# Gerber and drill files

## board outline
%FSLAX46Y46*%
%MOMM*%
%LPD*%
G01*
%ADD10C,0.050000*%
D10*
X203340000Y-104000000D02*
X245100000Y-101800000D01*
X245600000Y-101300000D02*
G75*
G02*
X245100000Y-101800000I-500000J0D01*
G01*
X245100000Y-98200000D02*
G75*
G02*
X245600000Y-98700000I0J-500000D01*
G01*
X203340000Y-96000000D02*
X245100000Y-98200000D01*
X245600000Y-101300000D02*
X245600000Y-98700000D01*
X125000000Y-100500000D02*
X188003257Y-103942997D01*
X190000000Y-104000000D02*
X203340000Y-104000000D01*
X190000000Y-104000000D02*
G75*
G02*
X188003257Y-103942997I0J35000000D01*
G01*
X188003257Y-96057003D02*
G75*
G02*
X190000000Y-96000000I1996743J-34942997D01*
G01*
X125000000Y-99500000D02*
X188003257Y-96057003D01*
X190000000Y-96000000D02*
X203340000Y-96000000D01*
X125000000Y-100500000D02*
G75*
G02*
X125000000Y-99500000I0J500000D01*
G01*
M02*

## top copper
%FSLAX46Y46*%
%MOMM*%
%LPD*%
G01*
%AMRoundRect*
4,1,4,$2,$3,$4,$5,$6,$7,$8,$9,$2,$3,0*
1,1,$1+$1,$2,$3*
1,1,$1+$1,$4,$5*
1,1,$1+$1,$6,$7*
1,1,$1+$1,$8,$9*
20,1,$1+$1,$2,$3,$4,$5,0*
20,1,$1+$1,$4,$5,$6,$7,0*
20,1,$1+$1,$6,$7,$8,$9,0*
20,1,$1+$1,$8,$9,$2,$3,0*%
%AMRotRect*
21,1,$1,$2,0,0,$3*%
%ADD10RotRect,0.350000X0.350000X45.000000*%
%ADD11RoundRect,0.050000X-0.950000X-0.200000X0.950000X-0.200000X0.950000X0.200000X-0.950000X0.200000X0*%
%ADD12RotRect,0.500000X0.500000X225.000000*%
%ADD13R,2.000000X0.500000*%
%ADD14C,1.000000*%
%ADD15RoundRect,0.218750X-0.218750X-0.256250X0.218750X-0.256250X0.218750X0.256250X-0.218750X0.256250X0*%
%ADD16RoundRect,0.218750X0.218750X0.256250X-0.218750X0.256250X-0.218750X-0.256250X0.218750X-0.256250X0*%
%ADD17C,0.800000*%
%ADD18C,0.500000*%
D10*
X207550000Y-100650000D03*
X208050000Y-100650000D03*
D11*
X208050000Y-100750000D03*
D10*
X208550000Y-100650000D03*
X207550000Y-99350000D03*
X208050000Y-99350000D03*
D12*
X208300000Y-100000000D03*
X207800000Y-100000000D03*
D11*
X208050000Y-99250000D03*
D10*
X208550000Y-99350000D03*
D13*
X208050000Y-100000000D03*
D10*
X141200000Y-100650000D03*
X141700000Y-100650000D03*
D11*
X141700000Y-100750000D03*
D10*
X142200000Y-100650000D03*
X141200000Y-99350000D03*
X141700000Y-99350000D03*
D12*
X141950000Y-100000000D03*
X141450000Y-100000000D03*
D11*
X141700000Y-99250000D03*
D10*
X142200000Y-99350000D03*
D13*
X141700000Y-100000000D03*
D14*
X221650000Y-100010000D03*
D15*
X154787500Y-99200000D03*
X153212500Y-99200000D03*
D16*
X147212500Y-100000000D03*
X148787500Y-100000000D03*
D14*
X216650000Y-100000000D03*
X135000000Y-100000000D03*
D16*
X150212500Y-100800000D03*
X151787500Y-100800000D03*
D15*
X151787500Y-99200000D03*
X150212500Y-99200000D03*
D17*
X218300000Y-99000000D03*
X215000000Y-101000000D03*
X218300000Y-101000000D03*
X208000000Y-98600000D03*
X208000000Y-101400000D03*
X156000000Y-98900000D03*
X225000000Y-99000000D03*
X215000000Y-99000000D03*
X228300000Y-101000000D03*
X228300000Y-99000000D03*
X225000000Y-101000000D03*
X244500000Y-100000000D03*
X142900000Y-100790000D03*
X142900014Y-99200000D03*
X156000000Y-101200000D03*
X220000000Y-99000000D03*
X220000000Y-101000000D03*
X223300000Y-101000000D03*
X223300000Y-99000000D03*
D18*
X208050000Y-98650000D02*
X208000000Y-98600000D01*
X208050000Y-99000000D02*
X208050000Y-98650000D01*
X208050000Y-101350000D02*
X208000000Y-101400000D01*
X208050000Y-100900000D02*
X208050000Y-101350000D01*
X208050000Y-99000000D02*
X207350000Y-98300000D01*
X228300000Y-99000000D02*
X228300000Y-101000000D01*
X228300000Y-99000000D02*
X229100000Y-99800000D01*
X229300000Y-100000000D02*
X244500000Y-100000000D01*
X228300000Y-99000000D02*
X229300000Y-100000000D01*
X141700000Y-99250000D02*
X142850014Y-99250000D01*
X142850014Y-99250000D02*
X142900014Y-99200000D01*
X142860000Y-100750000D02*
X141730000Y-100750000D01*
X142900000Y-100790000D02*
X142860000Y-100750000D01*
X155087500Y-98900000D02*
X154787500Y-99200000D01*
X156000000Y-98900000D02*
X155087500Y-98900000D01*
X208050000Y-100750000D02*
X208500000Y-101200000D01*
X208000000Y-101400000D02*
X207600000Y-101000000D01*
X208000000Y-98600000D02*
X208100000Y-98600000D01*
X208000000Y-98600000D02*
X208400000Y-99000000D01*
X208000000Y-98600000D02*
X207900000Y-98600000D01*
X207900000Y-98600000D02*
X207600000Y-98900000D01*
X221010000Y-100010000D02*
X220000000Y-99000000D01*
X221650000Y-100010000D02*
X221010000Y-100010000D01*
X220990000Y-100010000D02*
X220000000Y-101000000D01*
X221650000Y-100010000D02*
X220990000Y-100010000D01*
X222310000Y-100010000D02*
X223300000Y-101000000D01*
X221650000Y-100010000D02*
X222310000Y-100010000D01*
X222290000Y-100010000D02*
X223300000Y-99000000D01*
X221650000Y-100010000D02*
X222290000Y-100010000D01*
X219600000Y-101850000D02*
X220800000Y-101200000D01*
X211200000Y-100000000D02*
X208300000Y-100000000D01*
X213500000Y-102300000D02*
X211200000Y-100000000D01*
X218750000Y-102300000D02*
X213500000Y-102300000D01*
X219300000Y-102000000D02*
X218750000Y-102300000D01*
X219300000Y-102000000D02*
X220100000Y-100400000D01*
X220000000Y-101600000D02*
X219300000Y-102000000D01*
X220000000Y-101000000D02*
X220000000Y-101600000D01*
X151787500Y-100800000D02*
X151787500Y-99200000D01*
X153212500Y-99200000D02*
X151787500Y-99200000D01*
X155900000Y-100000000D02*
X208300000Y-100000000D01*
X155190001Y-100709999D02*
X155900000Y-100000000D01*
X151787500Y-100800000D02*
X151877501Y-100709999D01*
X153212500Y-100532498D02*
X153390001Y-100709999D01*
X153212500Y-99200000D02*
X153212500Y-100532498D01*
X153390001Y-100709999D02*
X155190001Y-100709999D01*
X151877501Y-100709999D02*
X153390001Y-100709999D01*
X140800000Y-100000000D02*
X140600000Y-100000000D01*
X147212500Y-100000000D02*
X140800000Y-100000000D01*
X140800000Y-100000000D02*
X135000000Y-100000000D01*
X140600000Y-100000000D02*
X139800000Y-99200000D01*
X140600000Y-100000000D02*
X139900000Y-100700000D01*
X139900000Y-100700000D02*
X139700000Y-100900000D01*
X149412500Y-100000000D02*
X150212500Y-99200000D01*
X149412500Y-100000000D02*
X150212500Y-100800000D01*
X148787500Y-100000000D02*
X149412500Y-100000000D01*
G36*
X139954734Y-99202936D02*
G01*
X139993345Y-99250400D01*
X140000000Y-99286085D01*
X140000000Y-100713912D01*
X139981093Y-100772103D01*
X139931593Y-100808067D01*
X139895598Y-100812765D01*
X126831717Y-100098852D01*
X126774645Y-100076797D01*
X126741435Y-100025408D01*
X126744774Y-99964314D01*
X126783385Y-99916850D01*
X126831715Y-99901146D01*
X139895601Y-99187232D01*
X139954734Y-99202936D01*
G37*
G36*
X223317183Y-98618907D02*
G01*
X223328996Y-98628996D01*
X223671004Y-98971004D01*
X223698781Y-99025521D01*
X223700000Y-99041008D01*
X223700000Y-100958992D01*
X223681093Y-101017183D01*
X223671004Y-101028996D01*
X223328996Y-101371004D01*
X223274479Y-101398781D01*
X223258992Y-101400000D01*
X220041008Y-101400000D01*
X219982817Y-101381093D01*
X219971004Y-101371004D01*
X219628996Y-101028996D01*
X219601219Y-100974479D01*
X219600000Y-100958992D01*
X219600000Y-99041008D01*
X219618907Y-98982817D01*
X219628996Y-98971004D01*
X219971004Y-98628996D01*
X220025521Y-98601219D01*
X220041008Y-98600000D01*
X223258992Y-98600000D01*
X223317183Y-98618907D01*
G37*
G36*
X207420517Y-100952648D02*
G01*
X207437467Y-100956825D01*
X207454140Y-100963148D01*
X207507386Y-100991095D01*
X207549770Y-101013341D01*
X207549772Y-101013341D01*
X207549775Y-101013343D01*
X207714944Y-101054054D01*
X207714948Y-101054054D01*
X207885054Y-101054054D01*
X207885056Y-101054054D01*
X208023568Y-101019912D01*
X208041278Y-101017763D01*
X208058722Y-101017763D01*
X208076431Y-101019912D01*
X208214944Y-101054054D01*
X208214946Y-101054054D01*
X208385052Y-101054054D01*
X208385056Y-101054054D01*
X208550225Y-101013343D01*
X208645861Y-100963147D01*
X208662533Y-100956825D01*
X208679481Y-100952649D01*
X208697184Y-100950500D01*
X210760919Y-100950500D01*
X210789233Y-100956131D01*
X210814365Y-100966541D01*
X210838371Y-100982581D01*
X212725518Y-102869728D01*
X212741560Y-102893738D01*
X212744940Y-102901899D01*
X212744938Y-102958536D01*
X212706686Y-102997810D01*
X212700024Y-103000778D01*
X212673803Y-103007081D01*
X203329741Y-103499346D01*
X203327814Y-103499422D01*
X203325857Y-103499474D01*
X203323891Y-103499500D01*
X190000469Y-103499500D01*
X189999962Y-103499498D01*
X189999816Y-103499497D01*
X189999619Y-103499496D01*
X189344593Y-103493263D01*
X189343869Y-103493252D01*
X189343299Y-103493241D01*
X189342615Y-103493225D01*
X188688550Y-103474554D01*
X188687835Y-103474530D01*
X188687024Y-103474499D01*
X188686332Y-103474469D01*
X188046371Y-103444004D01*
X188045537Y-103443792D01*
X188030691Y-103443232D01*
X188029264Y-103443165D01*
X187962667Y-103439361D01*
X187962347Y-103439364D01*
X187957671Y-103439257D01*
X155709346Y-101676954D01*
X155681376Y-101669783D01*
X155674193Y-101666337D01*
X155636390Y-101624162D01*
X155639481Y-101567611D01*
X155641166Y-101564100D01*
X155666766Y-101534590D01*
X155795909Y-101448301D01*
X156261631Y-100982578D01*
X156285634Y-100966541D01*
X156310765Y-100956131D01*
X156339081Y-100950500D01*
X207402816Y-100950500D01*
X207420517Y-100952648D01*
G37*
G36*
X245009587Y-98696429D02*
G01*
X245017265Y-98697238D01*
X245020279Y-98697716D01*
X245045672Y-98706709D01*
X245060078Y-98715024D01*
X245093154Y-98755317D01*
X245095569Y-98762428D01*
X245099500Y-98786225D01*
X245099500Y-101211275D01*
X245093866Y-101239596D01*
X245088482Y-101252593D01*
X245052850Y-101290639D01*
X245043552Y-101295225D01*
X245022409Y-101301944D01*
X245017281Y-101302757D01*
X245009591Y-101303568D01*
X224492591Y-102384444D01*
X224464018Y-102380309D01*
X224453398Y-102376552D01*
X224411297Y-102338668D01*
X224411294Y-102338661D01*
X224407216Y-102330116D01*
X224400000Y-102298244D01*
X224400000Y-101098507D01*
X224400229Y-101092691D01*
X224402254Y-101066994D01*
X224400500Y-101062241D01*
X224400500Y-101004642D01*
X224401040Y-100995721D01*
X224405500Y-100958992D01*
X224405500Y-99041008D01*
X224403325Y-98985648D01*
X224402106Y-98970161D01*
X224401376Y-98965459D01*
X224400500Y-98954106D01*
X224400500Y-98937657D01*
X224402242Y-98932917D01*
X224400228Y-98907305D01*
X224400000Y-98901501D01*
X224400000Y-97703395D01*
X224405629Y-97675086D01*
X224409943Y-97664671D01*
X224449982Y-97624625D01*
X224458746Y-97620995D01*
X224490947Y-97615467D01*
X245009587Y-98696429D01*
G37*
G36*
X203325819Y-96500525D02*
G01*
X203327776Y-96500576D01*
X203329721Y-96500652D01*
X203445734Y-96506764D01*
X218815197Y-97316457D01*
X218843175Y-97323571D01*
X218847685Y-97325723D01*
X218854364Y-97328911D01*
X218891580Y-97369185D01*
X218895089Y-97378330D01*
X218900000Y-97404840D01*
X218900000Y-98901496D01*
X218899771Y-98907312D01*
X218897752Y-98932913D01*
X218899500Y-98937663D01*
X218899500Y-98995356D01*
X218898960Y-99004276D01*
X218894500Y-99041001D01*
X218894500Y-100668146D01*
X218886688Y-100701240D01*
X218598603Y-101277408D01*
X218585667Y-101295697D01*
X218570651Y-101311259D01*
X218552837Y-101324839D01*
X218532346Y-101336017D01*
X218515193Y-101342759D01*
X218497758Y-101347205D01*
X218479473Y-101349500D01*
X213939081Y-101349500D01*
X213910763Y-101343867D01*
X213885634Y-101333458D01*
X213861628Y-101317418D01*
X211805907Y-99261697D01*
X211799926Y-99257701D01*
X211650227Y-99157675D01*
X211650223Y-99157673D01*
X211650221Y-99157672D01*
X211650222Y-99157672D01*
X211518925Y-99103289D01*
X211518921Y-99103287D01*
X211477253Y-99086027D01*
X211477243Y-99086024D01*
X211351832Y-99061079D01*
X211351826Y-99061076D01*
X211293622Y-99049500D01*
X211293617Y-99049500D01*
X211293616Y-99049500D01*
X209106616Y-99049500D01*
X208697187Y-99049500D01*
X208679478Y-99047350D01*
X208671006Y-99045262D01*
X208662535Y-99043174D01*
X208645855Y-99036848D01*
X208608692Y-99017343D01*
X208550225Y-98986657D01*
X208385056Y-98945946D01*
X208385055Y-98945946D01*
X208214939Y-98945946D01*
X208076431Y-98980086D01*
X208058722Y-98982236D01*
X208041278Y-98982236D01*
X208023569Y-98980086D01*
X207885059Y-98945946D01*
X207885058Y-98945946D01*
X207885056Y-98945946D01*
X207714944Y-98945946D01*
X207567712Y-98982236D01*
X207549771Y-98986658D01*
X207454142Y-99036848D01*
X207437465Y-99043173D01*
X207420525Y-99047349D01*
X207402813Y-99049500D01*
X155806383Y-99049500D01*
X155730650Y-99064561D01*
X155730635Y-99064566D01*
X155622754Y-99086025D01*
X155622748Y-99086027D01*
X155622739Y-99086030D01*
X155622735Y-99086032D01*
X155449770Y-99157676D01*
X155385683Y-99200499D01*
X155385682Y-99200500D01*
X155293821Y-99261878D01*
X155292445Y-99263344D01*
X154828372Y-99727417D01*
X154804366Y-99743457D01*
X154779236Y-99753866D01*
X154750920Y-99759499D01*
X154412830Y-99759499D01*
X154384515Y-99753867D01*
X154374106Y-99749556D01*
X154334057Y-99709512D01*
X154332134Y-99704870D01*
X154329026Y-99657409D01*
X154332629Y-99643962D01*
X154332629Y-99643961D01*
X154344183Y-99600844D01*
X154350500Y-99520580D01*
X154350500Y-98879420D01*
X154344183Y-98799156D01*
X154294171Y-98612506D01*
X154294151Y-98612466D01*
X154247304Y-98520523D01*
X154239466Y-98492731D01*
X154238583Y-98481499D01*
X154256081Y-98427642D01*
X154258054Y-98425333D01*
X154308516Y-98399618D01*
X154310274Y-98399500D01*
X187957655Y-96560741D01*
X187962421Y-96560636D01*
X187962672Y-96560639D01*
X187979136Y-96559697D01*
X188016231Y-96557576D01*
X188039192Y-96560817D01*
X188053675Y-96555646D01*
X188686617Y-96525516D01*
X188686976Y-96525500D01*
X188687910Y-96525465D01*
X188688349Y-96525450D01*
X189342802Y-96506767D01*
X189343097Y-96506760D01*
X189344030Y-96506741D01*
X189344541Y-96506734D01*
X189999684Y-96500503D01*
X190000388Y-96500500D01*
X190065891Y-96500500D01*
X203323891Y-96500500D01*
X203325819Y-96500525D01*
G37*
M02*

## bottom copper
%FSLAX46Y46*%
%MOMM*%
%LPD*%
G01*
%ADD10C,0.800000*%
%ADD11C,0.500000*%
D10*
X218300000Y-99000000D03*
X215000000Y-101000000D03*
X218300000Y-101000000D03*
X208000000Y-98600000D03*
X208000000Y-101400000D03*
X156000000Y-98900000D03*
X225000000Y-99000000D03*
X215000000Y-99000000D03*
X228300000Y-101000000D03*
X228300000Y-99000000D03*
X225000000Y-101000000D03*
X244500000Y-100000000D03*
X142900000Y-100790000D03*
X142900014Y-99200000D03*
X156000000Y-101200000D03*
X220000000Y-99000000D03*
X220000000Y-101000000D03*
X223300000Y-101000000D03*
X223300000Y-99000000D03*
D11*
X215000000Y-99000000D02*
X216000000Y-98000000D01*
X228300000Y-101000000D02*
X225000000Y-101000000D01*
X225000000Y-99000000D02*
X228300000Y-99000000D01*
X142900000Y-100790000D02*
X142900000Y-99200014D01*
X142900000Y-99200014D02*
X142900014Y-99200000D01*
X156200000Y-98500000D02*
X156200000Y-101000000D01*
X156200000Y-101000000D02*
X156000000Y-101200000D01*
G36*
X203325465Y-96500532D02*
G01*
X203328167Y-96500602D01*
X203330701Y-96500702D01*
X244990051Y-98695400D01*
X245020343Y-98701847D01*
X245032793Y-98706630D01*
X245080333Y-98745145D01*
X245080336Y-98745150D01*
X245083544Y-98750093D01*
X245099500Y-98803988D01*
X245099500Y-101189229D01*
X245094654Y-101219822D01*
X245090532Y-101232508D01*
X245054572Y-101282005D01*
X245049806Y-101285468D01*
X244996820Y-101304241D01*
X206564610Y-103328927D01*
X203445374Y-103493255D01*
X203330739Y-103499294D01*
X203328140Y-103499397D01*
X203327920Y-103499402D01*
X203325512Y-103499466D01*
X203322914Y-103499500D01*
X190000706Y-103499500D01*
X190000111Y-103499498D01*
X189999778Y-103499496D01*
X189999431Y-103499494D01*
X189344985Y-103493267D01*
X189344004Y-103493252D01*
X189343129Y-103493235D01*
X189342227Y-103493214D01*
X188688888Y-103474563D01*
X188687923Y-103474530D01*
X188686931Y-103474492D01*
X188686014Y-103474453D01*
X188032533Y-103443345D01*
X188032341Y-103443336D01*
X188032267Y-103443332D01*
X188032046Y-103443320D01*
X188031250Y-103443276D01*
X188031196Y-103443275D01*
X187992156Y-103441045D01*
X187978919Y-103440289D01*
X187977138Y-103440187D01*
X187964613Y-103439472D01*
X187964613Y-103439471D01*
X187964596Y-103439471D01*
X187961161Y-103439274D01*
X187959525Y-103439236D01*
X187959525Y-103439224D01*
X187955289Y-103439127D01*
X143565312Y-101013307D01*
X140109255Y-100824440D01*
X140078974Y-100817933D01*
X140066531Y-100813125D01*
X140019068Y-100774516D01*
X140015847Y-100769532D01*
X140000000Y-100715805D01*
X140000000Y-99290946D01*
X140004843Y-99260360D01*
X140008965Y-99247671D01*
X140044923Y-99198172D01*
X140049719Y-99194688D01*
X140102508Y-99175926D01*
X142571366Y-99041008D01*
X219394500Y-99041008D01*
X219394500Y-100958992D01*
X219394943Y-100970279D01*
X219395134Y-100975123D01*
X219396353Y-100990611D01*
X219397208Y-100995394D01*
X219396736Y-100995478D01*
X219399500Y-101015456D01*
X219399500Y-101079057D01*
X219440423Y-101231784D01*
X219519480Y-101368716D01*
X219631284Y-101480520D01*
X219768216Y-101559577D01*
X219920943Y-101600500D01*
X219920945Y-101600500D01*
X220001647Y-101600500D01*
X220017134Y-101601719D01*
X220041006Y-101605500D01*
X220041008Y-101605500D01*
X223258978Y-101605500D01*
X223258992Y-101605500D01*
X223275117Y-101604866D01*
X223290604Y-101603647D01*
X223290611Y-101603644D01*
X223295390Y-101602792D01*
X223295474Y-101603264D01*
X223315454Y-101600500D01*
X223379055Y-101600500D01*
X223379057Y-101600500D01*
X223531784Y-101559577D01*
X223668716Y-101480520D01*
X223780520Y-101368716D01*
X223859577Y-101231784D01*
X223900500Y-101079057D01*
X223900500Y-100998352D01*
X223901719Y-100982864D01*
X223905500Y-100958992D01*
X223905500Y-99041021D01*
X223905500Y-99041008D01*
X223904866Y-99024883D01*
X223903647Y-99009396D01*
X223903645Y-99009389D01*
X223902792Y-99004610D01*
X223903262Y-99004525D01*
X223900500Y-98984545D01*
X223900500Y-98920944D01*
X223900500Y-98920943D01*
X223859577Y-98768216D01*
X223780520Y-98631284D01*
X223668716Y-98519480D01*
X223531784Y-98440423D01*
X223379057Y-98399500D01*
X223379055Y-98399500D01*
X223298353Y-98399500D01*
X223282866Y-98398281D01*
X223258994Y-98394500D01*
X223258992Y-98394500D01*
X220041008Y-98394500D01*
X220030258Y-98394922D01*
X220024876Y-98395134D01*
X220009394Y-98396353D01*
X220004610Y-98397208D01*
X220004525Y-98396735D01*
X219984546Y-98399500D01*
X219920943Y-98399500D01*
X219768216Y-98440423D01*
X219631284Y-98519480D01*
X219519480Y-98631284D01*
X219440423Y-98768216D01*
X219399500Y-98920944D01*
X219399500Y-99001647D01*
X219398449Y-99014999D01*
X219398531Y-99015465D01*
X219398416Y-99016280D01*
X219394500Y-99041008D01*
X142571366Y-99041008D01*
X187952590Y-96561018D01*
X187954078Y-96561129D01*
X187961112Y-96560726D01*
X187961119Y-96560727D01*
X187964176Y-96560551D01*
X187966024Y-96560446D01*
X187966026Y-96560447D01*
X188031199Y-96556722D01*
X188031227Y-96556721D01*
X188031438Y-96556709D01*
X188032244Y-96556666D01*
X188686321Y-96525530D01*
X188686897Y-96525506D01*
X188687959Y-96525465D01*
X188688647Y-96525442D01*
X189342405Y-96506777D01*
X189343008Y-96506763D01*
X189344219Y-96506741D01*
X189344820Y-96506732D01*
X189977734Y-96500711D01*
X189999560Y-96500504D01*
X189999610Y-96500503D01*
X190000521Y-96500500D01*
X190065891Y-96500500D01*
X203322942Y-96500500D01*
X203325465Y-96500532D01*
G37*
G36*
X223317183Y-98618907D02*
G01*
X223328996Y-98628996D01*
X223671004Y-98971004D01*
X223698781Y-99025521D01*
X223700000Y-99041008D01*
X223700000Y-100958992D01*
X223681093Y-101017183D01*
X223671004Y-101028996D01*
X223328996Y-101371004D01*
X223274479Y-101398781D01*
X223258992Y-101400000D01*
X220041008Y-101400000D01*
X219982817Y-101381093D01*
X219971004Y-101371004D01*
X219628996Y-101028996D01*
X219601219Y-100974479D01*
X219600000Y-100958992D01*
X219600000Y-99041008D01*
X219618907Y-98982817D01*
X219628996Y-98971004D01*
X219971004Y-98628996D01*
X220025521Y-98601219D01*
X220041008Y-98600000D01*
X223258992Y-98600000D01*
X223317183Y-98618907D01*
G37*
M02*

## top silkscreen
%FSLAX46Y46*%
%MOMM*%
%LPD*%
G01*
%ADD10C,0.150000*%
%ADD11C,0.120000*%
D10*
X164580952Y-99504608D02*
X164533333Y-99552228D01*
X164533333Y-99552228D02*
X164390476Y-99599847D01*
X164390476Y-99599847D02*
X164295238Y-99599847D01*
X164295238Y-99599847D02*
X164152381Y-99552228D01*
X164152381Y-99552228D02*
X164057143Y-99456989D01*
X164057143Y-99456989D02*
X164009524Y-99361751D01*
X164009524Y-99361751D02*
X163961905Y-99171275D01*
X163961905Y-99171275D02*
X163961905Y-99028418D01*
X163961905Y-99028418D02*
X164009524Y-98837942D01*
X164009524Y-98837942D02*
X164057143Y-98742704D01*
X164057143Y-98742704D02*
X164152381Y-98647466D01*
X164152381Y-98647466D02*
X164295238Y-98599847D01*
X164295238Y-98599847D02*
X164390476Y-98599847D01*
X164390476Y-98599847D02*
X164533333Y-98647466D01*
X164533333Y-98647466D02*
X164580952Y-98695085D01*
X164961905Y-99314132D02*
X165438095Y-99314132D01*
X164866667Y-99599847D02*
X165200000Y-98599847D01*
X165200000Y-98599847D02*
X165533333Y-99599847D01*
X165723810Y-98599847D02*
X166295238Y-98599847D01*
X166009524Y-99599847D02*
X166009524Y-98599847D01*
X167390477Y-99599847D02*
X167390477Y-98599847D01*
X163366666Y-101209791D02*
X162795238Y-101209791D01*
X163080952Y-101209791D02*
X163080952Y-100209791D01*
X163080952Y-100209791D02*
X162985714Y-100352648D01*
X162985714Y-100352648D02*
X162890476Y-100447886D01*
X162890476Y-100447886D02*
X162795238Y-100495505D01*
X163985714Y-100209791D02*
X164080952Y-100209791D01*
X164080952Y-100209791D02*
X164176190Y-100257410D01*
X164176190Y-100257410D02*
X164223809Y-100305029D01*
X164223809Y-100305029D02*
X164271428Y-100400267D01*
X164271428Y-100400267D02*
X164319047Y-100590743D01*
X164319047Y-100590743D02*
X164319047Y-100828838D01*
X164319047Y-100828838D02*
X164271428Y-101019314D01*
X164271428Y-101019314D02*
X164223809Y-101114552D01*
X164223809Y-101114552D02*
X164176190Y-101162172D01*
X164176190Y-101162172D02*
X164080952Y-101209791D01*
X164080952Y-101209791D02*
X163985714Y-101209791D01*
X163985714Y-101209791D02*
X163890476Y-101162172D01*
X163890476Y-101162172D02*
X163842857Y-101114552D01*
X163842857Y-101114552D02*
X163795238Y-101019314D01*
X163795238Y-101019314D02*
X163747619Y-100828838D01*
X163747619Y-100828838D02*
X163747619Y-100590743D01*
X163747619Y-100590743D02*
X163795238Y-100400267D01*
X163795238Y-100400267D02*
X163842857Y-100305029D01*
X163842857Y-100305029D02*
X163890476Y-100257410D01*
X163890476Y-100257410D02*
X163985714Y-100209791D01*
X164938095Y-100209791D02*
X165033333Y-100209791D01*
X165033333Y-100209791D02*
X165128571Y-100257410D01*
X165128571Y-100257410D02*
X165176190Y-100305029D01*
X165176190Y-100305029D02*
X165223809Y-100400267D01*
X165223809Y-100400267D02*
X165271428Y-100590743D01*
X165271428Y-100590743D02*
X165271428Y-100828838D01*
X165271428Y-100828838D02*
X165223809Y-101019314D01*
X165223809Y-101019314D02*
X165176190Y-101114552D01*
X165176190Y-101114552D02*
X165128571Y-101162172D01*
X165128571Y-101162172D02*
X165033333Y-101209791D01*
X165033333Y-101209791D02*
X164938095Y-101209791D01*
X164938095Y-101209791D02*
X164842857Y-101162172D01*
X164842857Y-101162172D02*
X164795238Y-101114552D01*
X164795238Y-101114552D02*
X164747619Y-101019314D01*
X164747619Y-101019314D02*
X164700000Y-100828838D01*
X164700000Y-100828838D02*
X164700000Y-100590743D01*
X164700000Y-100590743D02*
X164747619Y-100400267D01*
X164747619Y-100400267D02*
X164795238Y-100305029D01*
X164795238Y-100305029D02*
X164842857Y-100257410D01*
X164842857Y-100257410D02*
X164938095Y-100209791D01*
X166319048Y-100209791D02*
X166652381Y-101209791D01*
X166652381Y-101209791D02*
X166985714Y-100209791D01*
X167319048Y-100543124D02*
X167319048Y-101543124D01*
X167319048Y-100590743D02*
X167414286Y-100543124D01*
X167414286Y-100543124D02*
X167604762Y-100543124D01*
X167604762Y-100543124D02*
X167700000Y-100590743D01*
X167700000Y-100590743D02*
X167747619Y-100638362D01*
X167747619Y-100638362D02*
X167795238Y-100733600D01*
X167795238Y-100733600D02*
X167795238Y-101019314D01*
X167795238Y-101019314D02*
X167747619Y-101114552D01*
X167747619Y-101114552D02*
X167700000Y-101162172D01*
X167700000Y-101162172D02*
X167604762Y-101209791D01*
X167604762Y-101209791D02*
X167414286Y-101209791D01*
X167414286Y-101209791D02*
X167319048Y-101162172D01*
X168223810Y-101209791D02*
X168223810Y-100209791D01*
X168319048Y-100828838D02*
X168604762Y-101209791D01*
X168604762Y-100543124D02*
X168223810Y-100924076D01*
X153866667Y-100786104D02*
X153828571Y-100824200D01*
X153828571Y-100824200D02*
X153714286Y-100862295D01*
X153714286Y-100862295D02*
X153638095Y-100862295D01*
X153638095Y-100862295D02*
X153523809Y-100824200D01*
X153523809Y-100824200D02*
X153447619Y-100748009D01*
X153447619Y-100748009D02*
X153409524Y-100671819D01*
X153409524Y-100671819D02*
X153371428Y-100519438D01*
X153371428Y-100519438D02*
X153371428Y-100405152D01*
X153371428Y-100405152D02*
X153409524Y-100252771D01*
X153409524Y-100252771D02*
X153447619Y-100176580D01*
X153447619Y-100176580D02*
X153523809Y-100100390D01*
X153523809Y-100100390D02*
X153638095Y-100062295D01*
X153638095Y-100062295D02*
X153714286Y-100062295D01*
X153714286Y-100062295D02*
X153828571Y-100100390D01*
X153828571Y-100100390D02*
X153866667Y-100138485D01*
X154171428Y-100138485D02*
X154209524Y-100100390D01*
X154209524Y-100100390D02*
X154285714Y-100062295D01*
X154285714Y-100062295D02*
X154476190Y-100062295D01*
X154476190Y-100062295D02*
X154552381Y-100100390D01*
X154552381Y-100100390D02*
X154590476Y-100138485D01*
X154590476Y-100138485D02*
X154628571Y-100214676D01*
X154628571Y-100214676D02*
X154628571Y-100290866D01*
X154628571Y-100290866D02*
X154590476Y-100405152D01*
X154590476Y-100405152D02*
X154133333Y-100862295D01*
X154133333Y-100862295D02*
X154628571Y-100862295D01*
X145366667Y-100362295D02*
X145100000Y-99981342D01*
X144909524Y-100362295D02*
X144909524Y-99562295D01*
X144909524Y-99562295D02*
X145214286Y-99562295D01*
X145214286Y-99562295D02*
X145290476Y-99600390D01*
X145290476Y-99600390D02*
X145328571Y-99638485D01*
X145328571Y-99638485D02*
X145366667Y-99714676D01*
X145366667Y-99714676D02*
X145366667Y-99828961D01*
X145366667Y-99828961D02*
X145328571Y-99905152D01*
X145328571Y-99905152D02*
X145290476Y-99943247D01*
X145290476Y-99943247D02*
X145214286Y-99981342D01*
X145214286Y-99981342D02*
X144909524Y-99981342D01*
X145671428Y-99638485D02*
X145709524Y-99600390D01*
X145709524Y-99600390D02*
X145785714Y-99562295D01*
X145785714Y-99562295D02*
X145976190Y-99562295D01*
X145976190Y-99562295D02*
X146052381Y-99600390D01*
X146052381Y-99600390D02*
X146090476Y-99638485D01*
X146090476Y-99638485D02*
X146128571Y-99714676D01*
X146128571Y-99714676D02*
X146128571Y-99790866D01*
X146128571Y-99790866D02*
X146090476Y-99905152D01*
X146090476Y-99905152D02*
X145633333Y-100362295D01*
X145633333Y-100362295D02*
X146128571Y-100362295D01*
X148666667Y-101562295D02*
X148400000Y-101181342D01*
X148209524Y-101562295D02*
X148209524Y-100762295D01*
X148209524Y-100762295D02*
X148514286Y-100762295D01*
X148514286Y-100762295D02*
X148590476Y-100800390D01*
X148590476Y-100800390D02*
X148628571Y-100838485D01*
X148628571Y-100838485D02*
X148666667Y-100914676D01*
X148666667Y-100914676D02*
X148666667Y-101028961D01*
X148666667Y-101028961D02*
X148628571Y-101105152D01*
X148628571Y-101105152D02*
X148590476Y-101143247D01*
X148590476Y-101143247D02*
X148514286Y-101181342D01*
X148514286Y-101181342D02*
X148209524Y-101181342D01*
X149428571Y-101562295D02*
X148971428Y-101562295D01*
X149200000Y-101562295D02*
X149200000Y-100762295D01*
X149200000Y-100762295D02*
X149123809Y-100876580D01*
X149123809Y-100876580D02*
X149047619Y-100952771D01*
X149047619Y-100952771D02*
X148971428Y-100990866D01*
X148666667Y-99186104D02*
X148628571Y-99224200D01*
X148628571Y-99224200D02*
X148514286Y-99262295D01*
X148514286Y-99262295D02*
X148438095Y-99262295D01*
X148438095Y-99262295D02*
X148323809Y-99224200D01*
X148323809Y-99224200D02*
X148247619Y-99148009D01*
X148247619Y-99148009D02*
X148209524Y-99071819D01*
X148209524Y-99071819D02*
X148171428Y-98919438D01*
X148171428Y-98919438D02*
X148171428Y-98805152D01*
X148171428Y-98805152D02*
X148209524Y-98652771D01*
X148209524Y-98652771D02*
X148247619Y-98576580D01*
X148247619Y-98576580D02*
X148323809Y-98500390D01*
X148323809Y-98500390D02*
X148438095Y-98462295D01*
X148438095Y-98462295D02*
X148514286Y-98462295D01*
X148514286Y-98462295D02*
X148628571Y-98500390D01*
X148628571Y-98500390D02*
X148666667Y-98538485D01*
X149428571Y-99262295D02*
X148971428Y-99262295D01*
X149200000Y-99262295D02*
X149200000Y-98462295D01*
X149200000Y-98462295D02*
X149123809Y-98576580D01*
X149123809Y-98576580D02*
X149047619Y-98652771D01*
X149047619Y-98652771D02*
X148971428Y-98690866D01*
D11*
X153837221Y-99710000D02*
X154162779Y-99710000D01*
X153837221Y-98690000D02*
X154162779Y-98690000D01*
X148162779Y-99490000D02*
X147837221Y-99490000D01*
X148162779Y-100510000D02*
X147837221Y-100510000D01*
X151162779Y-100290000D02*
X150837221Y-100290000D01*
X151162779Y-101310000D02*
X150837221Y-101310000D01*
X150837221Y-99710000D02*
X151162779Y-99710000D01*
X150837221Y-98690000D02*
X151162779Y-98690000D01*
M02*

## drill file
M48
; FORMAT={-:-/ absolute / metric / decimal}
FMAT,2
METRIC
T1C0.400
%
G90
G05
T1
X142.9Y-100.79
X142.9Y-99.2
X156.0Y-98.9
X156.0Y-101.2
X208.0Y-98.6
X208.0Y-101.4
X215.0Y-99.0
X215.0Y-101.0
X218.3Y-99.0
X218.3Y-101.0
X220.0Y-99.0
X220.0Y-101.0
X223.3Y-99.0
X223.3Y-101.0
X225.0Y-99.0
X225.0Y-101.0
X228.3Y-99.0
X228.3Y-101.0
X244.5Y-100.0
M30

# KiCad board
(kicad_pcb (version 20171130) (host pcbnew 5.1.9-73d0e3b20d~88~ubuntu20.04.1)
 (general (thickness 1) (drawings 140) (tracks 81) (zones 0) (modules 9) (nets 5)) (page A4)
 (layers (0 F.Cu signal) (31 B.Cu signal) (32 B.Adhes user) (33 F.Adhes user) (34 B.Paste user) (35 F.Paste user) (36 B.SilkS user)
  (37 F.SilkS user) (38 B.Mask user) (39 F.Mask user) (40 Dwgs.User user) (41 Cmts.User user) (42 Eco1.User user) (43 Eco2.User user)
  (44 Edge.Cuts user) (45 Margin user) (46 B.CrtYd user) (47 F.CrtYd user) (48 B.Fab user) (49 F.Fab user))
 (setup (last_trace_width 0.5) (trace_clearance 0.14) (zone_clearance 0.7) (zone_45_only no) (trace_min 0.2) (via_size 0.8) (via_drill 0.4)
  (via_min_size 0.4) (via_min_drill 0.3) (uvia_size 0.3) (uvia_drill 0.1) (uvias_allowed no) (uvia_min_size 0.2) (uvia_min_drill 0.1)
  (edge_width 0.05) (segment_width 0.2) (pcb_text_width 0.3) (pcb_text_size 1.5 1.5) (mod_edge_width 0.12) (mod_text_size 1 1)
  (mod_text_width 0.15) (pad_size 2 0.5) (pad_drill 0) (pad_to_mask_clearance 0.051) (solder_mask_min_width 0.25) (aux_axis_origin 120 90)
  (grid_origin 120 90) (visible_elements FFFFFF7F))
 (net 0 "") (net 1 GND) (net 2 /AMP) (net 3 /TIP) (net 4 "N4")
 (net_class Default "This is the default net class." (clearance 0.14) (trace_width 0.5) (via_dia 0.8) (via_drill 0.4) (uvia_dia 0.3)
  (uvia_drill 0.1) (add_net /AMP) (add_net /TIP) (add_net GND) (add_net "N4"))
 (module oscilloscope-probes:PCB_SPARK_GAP (layer F.Cu) (at 208.05 100)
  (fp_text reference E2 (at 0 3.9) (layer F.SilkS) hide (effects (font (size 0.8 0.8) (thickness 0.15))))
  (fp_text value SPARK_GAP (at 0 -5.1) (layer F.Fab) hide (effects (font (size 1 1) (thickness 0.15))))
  (pad 2 smd rect (at -0.5 0.65 45) (size 0.35 0.35) (layers F.Cu) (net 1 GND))
  (pad 2 smd rect (at 0 0.65 45) (size 0.35 0.35) (layers F.Cu) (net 1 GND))
  (pad 2 smd roundrect (at 0 0.75) (size 2 0.5) (layers F.Cu) (roundrect_rratio 0.1) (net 1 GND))
  (pad 2 smd rect (at 0.5 0.65 45) (size 0.35 0.35) (layers F.Cu) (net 1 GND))
  (pad 2 smd rect (at -0.5 -0.65 45) (size 0.35 0.35) (layers F.Cu) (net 1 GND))
  (pad 2 smd rect (at 0 -0.65 45) (size 0.35 0.35) (layers F.Cu) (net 1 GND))
  (pad 1 smd rect (at 0.25 0 225) (size 0.5 0.5) (layers F.Cu F.Mask) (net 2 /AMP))
  (pad 1 smd rect (at -0.25 0 225) (size 0.5 0.5) (layers F.Cu F.Mask) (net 2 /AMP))
  (pad 2 smd roundrect (at 0 -0.75) (size 2 0.5) (layers F.Cu) (roundrect_rratio 0.1) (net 1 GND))
  (pad 2 smd rect (at 0.5 -0.65 45) (size 0.35 0.35) (layers F.Cu) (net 1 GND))
  (pad 1 smd rect (at 0 0) (size 2 0.5) (layers F.Cu F.Mask) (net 2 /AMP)))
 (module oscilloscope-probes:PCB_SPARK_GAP (layer F.Cu) (at 141.7 100)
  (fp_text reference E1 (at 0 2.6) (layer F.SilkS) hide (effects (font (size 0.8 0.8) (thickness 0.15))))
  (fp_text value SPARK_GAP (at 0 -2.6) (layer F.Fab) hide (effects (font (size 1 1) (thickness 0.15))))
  (pad 2 smd rect (at -0.5 0.65 45) (size 0.35 0.35) (layers F.Cu) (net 1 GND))
  (pad 2 smd rect (at 0 0.65 45) (size 0.35 0.35) (layers F.Cu) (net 1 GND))
  (pad 2 smd roundrect (at 0 0.75) (size 2 0.5) (layers F.Cu) (roundrect_rratio 0.1) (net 1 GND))
  (pad 2 smd rect (at 0.5 0.65 45) (size 0.35 0.35) (layers F.Cu) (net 1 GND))
  (pad 2 smd rect (at -0.5 -0.65 45) (size 0.35 0.35) (layers F.Cu) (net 1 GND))
  (pad 2 smd rect (at 0 -0.65 45) (size 0.35 0.35) (layers F.Cu) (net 1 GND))
  (pad 1 smd rect (at 0.25 0 225) (size 0.5 0.5) (layers F.Cu F.Mask) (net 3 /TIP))
  (pad 1 smd rect (at -0.25 0 225) (size 0.5 0.5) (layers F.Cu F.Mask) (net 3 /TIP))
  (pad 2 smd roundrect (at 0 -0.75) (size 2 0.5) (layers F.Cu) (roundrect_rratio 0.1) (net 1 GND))
  (pad 2 smd rect (at 0.5 -0.65 45) (size 0.35 0.35) (layers F.Cu) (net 1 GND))
  (pad 1 smd rect (at 0 0) (size 2 0.5) (layers F.Cu F.Mask) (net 3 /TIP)))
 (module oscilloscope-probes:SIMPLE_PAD (layer F.Cu) (at 221.65 100.01)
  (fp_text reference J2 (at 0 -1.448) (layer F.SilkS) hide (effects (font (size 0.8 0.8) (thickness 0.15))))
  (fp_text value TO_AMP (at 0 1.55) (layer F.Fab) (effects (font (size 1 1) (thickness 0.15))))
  (pad 1 smd circle (at 0 0) (size 1 1) (layers F.Cu F.Mask) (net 2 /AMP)))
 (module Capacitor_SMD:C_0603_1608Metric (layer F.Cu) (at 154 99.2)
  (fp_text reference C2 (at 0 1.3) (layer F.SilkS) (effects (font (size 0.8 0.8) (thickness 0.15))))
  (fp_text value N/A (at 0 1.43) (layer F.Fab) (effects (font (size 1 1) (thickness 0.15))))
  (fp_line (start -0.162779 0.51) (end 0.162779 0.51) (layer F.SilkS) (width 0.12))
  (fp_line (start -0.162779 -0.51) (end 0.162779 -0.51) (layer F.SilkS) (width 0.12))
  (pad 2 smd roundrect (at 0.7875 0) (size 0.875 0.95) (layers F.Cu F.Paste F.Mask) (roundrect_rratio 0.25) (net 1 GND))
  (pad 1 smd roundrect (at -0.7875 0) (size 0.875 0.95) (layers F.Cu F.Paste F.Mask) (roundrect_rratio 0.25) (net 2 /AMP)))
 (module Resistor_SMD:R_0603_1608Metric (layer F.Cu) (at 148 100 180)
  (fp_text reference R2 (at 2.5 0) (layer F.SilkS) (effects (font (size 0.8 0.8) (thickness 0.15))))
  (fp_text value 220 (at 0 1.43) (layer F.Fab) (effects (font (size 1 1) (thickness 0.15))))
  (fp_line (start -0.162779 0.51) (end 0.162779 0.51) (layer F.SilkS) (width 0.12))
  (fp_line (start -0.162779 -0.51) (end 0.162779 -0.51) (layer F.SilkS) (width 0.12))
  (pad 2 smd roundrect (at 0.7875 0 180) (size 0.875 0.95) (layers F.Cu F.Paste F.Mask) (roundrect_rratio 0.25) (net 3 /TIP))
  (pad 1 smd roundrect (at -0.7875 0 180) (size 0.875 0.95) (layers F.Cu F.Paste F.Mask) (roundrect_rratio 0.25) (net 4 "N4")))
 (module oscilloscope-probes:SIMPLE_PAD (layer F.Cu) (at 216.65 100)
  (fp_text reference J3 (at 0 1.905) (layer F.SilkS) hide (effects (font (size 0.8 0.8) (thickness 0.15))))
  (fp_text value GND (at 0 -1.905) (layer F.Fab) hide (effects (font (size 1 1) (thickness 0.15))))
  (pad 1 smd circle (at 0 0) (size 1 1) (layers F.Cu F.Mask) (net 1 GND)))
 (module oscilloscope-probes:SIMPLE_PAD (layer F.Cu) (at 135 100)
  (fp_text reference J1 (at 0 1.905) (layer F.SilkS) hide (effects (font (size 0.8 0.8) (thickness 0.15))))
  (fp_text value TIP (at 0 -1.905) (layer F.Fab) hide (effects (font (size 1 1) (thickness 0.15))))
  (pad 1 smd circle (at 0 0) (size 1 1) (layers F.Cu F.Mask) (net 3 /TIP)))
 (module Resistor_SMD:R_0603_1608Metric (layer F.Cu) (at 151 100.8 180)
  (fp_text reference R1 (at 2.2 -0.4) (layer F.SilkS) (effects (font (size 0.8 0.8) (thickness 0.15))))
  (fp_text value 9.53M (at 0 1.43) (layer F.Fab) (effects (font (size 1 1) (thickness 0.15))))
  (fp_line (start -0.162779 0.51) (end 0.162779 0.51) (layer F.SilkS) (width 0.12))
  (fp_line (start -0.162779 -0.51) (end 0.162779 -0.51) (layer F.SilkS) (width 0.12))
  (pad 2 smd roundrect (at 0.7875 0 180) (size 0.875 0.95) (layers F.Cu F.Paste F.Mask) (roundrect_rratio 0.25) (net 4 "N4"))
  (pad 1 smd roundrect (at -0.7875 0 180) (size 0.875 0.95) (layers F.Cu F.Paste F.Mask) (roundrect_rratio 0.25) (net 2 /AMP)))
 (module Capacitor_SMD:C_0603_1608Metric (layer F.Cu) (at 151 99.2)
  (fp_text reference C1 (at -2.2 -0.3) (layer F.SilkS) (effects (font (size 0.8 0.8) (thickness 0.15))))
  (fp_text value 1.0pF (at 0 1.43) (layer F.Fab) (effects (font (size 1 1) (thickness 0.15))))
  (fp_line (start -0.162779 0.51) (end 0.162779 0.51) (layer F.SilkS) (width 0.12))
  (fp_line (start -0.162779 -0.51) (end 0.162779 -0.51) (layer F.SilkS) (width 0.12))
  (pad 2 smd roundrect (at 0.7875 0) (size 0.875 0.95) (layers F.Cu F.Paste F.Mask) (roundrect_rratio 0.25) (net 2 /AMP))
  (pad 1 smd roundrect (at -0.7875 0) (size 0.875 0.95) (layers F.Cu F.Paste F.Mask) (roundrect_rratio 0.25) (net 4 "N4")))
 (gr_line (start 203.34 104) (end 245.1 101.8) (layer Edge.Cuts) (width 0.05))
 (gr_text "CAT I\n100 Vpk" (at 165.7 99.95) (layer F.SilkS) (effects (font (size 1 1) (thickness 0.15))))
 (gr_arc (start 245.1 101.3) (end 245.1 101.8) (angle -90) (layer Edge.Cuts) (width 0.05))
 (gr_arc (start 245.1 98.7) (end 245.6 98.7) (angle -90) (layer Edge.Cuts) (width 0.05))
 (gr_line (start 203.34 96) (end 245.1 98.2) (layer Edge.Cuts) (width 0.05))
 (gr_line (start 245.6 101.3) (end 245.6 98.7) (layer Edge.Cuts) (width 0.05))
 (gr_line (start 125 100.5) (end 188.003257 103.942997) (layer Edge.Cuts) (width 0.05))
 (gr_line (start 190 104) (end 203.34 104) (layer Edge.Cuts) (width 0.05))
 (gr_arc (start 190 69) (end 190 104) (angle 3.270487923) (layer Edge.Cuts) (width 0.05))
 (gr_arc (start 190 131) (end 190 96) (angle -3.270487923) (layer Edge.Cuts) (width 0.05))
 (gr_line (start 125 99.5) (end 188.003257 96.057003) (layer Edge.Cuts) (width 0.05))
 (gr_line (start 190 96) (end 203.34 96) (layer Edge.Cuts) (width 0.05))
 (gr_arc (start 125 100) (end 125 99.5) (angle -180) (layer Edge.Cuts) (width 0.05))
 (via (at 218.3 99) (size 0.8) (drill 0.4) (layers F.Cu B.Cu) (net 1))
 (via (at 215 101) (size 0.8) (drill 0.4) (layers F.Cu B.Cu) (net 1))
 (via (at 218.3 101) (size 0.8) (drill 0.4) (layers F.Cu B.Cu) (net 1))
 (via (at 208 98.6) (size 0.8) (drill 0.4) (layers F.Cu B.Cu) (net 1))
 (segment (start 208.05 98.65) (end 208 98.6) (width 0.5) (layer F.Cu) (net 1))
 (segment (start 208.05 99) (end 208.05 98.65) (width 0.5) (layer F.Cu) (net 1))
 (via (at 208 101.4) (size 0.8) (drill 0.4) (layers F.Cu B.Cu) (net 1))
 (segment (start 208.05 101.35) (end 208 101.4) (width 0.5) (layer F.Cu) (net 1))
 (segment (start 208.05 100.9) (end 208.05 101.35) (width 0.5) (layer F.Cu) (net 1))
 (segment (start 208.05 99) (end 207.35 98.3) (width 0.5) (layer F.Cu) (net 1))
 (via (at 156 98.9) (size 0.8) (drill 0.4) (layers F.Cu B.Cu) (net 1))
 (via (at 225 99) (size 0.8) (drill 0.4) (layers F.Cu B.Cu) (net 1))
 (segment (start 215 99) (end 216 98) (width 0.5) (layer B.Cu) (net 1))
 (via (at 215 99) (size 0.8) (drill 0.4) (layers F.Cu B.Cu) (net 1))
 (segment (start 228.3 101) (end 225 101) (width 0.5) (layer B.Cu) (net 1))
 (via (at 228.3 101) (size 0.8) (drill 0.4) (layers F.Cu B.Cu) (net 1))
 (via (at 228.3 99) (size 0.8) (drill 0.4) (layers F.Cu B.Cu) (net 1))
 (segment (start 225 99) (end 228.3 99) (width 0.5) (layer B.Cu) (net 1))
 (via (at 225 101) (size 0.8) (drill 0.4) (layers F.Cu B.Cu) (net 1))
 (segment (start 228.3 99) (end 228.3 101) (width 0.5) (layer F.Cu) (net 1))
 (segment (start 228.3 99) (end 229.1 99.8) (width 0.5) (layer F.Cu) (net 1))
 (via (at 244.5 100) (size 0.8) (drill 0.4) (layers F.Cu B.Cu) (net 1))
 (segment (start 229.3 100) (end 244.5 100) (width 0.5) (layer F.Cu) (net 1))
 (segment (start 228.3 99) (end 229.3 100) (width 0.5) (layer F.Cu) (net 1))
 (via (at 142.9 100.79) (size 0.8) (drill 0.4) (layers F.Cu B.Cu) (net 1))
 (via (at 142.900014 99.2) (size 0.8) (drill 0.4) (layers F.Cu B.Cu) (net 1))
 (segment (start 142.9 100.79) (end 142.9 99.200014) (width 0.5) (layer B.Cu) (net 1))
 (segment (start 142.9 99.200014) (end 142.900014 99.2) (width 0.5) (layer B.Cu) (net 1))
 (segment (start 141.7 99.25) (end 142.850014 99.25) (width 0.5) (layer F.Cu) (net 1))
 (segment (start 142.850014 99.25) (end 142.900014 99.2) (width 0.5) (layer F.Cu) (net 1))
 (segment (start 142.86 100.75) (end 141.73 100.75) (width 0.5) (layer F.Cu) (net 1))
 (segment (start 142.9 100.79) (end 142.86 100.75) (width 0.5) (layer F.Cu) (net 1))
 (segment (start 155.0875 98.9) (end 154.7875 99.2) (width 0.5) (layer F.Cu) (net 1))
 (segment (start 156 98.9) (end 155.0875 98.9) (width 0.5) (layer F.Cu) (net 1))
 (via (at 156 101.2) (size 0.8) (drill 0.4) (layers F.Cu B.Cu) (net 1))
 (segment (start 156.2 98.5) (end 156.2 101) (width 0.5) (layer B.Cu) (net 1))
 (segment (start 156.2 101) (end 156 101.2) (width 0.5) (layer B.Cu) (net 1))
 (segment (start 208.05 100.75) (end 208.5 101.2) (width 0.5) (layer F.Cu) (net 1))
 (segment (start 208 101.4) (end 207.6 101) (width 0.5) (layer F.Cu) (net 1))
 (segment (start 208 98.6) (end 208.1 98.6) (width 0.5) (layer F.Cu) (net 1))
 (segment (start 208 98.6) (end 208.4 99) (width 0.5) (layer F.Cu) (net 1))
 (segment (start 208 98.6) (end 207.9 98.6) (width 0.5) (layer F.Cu) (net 1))
 (segment (start 207.9 98.6) (end 207.6 98.9) (width 0.5) (layer F.Cu) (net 1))
 (via (at 220 99) (size 0.8) (drill 0.4) (layers F.Cu B.Cu) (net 2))
 (segment (start 221.01 100.01) (end 220 99) (width 0.5) (layer F.Cu) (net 2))
 (segment (start 221.65 100.01) (end 221.01 100.01) (width 0.5) (layer F.Cu) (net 2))
 (via (at 220 101) (size 0.8) (drill 0.4) (layers F.Cu B.Cu) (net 2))
 (segment (start 220.99 100.01) (end 220 101) (width 0.5) (layer F.Cu) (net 2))
 (segment (start 221.65 100.01) (end 220.99 100.01) (width 0.5) (layer F.Cu) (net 2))
 (via (at 223.3 101) (size 0.8) (drill 0.4) (layers F.Cu B.Cu) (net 2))
 (segment (start 222.31 100.01) (end 223.3 101) (width 0.5) (layer F.Cu) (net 2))
 (segment (start 221.65 100.01) (end 222.31 100.01) (width 0.5) (layer F.Cu) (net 2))
 (via (at 223.3 99) (size 0.8) (drill 0.4) (layers F.Cu B.Cu) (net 2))
 (segment (start 222.29 100.01) (end 223.3 99) (width 0.5) (layer F.Cu) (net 2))
 (segment (start 221.65 100.01) (end 222.29 100.01) (width 0.5) (layer F.Cu) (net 2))
 (segment (start 219.6 101.85) (end 220.8 101.2) (width 0.5) (layer F.Cu) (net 2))
 (segment (start 211.2 100) (end 208.3 100) (width 0.5) (layer F.Cu) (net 2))
 (segment (start 213.5 102.3) (end 211.2 100) (width 0.5) (layer F.Cu) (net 2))
 (segment (start 218.75 102.3) (end 213.5 102.3) (width 0.5) (layer F.Cu) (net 2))
 (segment (start 219.3 102) (end 218.75 102.3) (width 0.5) (layer F.Cu) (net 2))
 (segment (start 219.3 102) (end 220.1 100.4) (width 0.5) (layer F.Cu) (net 2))
 (segment (start 220 101.6) (end 219.3 102) (width 0.5) (layer F.Cu) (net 2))
 (segment (start 220 101) (end 220 101.6) (width 0.5) (layer F.Cu) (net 2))
 (segment (start 151.7875 100.8) (end 151.7875 99.2) (width 0.5) (layer F.Cu) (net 2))
 (segment (start 153.2125 99.2) (end 151.7875 99.2) (width 0.5) (layer F.Cu) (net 2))
 (segment (start 155.9 100) (end 208.3 100) (width 0.5) (layer F.Cu) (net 2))
 (segment (start 155.190001 100.709999) (end 155.9 100) (width 0.5) (layer F.Cu) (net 2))
 (segment (start 151.7875 100.8) (end 151.877501 100.709999) (width 0.5) (layer F.Cu) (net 2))
 (segment (start 153.2125 100.532498) (end 153.390001 100.709999) (width 0.5) (layer F.Cu) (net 2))
 (segment (start 153.2125 99.2) (end 153.2125 100.532498) (width 0.5) (layer F.Cu) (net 2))
 (segment (start 153.390001 100.709999) (end 155.190001 100.709999) (width 0.5) (layer F.Cu) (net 2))
 (segment (start 151.877501 100.709999) (end 153.390001 100.709999) (width 0.5) (layer F.Cu) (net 2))
 (segment (start 140.8 100) (end 140.6 100) (width 0.5) (layer F.Cu) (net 3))
 (segment (start 147.2125 100) (end 140.8 100) (width 0.5) (layer F.Cu) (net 3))
 (segment (start 140.8 100) (end 135 100) (width 0.5) (layer F.Cu) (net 3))
 (segment (start 140.6 100) (end 139.8 99.2) (width 0.5) (layer F.Cu) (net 3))
 (segment (start 140.6 100) (end 139.9 100.7) (width 0.5) (layer F.Cu) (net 3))
 (segment (start 139.9 100.7) (end 139.7 100.9) (width 0.5) (layer F.Cu) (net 3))
 (segment (start 149.4125 100) (end 150.2125 99.2) (width 0.5) (layer F.Cu) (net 4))
 (segment (start 149.4125 100) (end 150.2125 100.8) (width 0.5) (layer F.Cu) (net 4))
 (segment (start 148.7875 100) (end 149.4125 100) (width 0.5) (layer F.Cu) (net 4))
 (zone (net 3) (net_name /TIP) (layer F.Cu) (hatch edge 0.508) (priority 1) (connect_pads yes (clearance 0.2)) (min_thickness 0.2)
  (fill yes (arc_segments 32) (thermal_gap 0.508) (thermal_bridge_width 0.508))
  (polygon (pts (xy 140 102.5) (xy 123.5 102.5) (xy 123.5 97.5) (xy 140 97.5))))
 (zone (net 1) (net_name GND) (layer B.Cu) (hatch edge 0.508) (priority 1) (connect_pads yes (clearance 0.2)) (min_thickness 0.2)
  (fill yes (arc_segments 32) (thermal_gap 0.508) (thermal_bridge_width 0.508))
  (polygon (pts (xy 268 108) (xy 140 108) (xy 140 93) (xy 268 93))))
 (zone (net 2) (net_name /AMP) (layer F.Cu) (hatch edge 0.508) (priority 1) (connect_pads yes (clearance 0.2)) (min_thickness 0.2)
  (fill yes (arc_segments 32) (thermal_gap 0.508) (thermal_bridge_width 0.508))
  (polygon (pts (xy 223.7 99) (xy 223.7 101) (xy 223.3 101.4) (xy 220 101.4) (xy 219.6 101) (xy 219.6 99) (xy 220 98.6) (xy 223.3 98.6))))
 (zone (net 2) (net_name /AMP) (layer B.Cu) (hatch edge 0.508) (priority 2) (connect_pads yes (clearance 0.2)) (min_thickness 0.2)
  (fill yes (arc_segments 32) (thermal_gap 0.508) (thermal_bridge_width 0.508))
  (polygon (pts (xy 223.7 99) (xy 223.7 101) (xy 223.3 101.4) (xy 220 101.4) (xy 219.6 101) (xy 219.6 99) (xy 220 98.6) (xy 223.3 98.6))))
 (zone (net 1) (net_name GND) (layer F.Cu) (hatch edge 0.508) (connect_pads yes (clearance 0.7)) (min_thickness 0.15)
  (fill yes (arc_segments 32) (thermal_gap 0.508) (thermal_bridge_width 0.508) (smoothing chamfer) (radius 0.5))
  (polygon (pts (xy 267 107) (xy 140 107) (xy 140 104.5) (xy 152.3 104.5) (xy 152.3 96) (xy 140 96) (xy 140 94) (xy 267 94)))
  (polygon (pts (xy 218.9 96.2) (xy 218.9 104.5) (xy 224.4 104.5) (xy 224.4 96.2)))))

